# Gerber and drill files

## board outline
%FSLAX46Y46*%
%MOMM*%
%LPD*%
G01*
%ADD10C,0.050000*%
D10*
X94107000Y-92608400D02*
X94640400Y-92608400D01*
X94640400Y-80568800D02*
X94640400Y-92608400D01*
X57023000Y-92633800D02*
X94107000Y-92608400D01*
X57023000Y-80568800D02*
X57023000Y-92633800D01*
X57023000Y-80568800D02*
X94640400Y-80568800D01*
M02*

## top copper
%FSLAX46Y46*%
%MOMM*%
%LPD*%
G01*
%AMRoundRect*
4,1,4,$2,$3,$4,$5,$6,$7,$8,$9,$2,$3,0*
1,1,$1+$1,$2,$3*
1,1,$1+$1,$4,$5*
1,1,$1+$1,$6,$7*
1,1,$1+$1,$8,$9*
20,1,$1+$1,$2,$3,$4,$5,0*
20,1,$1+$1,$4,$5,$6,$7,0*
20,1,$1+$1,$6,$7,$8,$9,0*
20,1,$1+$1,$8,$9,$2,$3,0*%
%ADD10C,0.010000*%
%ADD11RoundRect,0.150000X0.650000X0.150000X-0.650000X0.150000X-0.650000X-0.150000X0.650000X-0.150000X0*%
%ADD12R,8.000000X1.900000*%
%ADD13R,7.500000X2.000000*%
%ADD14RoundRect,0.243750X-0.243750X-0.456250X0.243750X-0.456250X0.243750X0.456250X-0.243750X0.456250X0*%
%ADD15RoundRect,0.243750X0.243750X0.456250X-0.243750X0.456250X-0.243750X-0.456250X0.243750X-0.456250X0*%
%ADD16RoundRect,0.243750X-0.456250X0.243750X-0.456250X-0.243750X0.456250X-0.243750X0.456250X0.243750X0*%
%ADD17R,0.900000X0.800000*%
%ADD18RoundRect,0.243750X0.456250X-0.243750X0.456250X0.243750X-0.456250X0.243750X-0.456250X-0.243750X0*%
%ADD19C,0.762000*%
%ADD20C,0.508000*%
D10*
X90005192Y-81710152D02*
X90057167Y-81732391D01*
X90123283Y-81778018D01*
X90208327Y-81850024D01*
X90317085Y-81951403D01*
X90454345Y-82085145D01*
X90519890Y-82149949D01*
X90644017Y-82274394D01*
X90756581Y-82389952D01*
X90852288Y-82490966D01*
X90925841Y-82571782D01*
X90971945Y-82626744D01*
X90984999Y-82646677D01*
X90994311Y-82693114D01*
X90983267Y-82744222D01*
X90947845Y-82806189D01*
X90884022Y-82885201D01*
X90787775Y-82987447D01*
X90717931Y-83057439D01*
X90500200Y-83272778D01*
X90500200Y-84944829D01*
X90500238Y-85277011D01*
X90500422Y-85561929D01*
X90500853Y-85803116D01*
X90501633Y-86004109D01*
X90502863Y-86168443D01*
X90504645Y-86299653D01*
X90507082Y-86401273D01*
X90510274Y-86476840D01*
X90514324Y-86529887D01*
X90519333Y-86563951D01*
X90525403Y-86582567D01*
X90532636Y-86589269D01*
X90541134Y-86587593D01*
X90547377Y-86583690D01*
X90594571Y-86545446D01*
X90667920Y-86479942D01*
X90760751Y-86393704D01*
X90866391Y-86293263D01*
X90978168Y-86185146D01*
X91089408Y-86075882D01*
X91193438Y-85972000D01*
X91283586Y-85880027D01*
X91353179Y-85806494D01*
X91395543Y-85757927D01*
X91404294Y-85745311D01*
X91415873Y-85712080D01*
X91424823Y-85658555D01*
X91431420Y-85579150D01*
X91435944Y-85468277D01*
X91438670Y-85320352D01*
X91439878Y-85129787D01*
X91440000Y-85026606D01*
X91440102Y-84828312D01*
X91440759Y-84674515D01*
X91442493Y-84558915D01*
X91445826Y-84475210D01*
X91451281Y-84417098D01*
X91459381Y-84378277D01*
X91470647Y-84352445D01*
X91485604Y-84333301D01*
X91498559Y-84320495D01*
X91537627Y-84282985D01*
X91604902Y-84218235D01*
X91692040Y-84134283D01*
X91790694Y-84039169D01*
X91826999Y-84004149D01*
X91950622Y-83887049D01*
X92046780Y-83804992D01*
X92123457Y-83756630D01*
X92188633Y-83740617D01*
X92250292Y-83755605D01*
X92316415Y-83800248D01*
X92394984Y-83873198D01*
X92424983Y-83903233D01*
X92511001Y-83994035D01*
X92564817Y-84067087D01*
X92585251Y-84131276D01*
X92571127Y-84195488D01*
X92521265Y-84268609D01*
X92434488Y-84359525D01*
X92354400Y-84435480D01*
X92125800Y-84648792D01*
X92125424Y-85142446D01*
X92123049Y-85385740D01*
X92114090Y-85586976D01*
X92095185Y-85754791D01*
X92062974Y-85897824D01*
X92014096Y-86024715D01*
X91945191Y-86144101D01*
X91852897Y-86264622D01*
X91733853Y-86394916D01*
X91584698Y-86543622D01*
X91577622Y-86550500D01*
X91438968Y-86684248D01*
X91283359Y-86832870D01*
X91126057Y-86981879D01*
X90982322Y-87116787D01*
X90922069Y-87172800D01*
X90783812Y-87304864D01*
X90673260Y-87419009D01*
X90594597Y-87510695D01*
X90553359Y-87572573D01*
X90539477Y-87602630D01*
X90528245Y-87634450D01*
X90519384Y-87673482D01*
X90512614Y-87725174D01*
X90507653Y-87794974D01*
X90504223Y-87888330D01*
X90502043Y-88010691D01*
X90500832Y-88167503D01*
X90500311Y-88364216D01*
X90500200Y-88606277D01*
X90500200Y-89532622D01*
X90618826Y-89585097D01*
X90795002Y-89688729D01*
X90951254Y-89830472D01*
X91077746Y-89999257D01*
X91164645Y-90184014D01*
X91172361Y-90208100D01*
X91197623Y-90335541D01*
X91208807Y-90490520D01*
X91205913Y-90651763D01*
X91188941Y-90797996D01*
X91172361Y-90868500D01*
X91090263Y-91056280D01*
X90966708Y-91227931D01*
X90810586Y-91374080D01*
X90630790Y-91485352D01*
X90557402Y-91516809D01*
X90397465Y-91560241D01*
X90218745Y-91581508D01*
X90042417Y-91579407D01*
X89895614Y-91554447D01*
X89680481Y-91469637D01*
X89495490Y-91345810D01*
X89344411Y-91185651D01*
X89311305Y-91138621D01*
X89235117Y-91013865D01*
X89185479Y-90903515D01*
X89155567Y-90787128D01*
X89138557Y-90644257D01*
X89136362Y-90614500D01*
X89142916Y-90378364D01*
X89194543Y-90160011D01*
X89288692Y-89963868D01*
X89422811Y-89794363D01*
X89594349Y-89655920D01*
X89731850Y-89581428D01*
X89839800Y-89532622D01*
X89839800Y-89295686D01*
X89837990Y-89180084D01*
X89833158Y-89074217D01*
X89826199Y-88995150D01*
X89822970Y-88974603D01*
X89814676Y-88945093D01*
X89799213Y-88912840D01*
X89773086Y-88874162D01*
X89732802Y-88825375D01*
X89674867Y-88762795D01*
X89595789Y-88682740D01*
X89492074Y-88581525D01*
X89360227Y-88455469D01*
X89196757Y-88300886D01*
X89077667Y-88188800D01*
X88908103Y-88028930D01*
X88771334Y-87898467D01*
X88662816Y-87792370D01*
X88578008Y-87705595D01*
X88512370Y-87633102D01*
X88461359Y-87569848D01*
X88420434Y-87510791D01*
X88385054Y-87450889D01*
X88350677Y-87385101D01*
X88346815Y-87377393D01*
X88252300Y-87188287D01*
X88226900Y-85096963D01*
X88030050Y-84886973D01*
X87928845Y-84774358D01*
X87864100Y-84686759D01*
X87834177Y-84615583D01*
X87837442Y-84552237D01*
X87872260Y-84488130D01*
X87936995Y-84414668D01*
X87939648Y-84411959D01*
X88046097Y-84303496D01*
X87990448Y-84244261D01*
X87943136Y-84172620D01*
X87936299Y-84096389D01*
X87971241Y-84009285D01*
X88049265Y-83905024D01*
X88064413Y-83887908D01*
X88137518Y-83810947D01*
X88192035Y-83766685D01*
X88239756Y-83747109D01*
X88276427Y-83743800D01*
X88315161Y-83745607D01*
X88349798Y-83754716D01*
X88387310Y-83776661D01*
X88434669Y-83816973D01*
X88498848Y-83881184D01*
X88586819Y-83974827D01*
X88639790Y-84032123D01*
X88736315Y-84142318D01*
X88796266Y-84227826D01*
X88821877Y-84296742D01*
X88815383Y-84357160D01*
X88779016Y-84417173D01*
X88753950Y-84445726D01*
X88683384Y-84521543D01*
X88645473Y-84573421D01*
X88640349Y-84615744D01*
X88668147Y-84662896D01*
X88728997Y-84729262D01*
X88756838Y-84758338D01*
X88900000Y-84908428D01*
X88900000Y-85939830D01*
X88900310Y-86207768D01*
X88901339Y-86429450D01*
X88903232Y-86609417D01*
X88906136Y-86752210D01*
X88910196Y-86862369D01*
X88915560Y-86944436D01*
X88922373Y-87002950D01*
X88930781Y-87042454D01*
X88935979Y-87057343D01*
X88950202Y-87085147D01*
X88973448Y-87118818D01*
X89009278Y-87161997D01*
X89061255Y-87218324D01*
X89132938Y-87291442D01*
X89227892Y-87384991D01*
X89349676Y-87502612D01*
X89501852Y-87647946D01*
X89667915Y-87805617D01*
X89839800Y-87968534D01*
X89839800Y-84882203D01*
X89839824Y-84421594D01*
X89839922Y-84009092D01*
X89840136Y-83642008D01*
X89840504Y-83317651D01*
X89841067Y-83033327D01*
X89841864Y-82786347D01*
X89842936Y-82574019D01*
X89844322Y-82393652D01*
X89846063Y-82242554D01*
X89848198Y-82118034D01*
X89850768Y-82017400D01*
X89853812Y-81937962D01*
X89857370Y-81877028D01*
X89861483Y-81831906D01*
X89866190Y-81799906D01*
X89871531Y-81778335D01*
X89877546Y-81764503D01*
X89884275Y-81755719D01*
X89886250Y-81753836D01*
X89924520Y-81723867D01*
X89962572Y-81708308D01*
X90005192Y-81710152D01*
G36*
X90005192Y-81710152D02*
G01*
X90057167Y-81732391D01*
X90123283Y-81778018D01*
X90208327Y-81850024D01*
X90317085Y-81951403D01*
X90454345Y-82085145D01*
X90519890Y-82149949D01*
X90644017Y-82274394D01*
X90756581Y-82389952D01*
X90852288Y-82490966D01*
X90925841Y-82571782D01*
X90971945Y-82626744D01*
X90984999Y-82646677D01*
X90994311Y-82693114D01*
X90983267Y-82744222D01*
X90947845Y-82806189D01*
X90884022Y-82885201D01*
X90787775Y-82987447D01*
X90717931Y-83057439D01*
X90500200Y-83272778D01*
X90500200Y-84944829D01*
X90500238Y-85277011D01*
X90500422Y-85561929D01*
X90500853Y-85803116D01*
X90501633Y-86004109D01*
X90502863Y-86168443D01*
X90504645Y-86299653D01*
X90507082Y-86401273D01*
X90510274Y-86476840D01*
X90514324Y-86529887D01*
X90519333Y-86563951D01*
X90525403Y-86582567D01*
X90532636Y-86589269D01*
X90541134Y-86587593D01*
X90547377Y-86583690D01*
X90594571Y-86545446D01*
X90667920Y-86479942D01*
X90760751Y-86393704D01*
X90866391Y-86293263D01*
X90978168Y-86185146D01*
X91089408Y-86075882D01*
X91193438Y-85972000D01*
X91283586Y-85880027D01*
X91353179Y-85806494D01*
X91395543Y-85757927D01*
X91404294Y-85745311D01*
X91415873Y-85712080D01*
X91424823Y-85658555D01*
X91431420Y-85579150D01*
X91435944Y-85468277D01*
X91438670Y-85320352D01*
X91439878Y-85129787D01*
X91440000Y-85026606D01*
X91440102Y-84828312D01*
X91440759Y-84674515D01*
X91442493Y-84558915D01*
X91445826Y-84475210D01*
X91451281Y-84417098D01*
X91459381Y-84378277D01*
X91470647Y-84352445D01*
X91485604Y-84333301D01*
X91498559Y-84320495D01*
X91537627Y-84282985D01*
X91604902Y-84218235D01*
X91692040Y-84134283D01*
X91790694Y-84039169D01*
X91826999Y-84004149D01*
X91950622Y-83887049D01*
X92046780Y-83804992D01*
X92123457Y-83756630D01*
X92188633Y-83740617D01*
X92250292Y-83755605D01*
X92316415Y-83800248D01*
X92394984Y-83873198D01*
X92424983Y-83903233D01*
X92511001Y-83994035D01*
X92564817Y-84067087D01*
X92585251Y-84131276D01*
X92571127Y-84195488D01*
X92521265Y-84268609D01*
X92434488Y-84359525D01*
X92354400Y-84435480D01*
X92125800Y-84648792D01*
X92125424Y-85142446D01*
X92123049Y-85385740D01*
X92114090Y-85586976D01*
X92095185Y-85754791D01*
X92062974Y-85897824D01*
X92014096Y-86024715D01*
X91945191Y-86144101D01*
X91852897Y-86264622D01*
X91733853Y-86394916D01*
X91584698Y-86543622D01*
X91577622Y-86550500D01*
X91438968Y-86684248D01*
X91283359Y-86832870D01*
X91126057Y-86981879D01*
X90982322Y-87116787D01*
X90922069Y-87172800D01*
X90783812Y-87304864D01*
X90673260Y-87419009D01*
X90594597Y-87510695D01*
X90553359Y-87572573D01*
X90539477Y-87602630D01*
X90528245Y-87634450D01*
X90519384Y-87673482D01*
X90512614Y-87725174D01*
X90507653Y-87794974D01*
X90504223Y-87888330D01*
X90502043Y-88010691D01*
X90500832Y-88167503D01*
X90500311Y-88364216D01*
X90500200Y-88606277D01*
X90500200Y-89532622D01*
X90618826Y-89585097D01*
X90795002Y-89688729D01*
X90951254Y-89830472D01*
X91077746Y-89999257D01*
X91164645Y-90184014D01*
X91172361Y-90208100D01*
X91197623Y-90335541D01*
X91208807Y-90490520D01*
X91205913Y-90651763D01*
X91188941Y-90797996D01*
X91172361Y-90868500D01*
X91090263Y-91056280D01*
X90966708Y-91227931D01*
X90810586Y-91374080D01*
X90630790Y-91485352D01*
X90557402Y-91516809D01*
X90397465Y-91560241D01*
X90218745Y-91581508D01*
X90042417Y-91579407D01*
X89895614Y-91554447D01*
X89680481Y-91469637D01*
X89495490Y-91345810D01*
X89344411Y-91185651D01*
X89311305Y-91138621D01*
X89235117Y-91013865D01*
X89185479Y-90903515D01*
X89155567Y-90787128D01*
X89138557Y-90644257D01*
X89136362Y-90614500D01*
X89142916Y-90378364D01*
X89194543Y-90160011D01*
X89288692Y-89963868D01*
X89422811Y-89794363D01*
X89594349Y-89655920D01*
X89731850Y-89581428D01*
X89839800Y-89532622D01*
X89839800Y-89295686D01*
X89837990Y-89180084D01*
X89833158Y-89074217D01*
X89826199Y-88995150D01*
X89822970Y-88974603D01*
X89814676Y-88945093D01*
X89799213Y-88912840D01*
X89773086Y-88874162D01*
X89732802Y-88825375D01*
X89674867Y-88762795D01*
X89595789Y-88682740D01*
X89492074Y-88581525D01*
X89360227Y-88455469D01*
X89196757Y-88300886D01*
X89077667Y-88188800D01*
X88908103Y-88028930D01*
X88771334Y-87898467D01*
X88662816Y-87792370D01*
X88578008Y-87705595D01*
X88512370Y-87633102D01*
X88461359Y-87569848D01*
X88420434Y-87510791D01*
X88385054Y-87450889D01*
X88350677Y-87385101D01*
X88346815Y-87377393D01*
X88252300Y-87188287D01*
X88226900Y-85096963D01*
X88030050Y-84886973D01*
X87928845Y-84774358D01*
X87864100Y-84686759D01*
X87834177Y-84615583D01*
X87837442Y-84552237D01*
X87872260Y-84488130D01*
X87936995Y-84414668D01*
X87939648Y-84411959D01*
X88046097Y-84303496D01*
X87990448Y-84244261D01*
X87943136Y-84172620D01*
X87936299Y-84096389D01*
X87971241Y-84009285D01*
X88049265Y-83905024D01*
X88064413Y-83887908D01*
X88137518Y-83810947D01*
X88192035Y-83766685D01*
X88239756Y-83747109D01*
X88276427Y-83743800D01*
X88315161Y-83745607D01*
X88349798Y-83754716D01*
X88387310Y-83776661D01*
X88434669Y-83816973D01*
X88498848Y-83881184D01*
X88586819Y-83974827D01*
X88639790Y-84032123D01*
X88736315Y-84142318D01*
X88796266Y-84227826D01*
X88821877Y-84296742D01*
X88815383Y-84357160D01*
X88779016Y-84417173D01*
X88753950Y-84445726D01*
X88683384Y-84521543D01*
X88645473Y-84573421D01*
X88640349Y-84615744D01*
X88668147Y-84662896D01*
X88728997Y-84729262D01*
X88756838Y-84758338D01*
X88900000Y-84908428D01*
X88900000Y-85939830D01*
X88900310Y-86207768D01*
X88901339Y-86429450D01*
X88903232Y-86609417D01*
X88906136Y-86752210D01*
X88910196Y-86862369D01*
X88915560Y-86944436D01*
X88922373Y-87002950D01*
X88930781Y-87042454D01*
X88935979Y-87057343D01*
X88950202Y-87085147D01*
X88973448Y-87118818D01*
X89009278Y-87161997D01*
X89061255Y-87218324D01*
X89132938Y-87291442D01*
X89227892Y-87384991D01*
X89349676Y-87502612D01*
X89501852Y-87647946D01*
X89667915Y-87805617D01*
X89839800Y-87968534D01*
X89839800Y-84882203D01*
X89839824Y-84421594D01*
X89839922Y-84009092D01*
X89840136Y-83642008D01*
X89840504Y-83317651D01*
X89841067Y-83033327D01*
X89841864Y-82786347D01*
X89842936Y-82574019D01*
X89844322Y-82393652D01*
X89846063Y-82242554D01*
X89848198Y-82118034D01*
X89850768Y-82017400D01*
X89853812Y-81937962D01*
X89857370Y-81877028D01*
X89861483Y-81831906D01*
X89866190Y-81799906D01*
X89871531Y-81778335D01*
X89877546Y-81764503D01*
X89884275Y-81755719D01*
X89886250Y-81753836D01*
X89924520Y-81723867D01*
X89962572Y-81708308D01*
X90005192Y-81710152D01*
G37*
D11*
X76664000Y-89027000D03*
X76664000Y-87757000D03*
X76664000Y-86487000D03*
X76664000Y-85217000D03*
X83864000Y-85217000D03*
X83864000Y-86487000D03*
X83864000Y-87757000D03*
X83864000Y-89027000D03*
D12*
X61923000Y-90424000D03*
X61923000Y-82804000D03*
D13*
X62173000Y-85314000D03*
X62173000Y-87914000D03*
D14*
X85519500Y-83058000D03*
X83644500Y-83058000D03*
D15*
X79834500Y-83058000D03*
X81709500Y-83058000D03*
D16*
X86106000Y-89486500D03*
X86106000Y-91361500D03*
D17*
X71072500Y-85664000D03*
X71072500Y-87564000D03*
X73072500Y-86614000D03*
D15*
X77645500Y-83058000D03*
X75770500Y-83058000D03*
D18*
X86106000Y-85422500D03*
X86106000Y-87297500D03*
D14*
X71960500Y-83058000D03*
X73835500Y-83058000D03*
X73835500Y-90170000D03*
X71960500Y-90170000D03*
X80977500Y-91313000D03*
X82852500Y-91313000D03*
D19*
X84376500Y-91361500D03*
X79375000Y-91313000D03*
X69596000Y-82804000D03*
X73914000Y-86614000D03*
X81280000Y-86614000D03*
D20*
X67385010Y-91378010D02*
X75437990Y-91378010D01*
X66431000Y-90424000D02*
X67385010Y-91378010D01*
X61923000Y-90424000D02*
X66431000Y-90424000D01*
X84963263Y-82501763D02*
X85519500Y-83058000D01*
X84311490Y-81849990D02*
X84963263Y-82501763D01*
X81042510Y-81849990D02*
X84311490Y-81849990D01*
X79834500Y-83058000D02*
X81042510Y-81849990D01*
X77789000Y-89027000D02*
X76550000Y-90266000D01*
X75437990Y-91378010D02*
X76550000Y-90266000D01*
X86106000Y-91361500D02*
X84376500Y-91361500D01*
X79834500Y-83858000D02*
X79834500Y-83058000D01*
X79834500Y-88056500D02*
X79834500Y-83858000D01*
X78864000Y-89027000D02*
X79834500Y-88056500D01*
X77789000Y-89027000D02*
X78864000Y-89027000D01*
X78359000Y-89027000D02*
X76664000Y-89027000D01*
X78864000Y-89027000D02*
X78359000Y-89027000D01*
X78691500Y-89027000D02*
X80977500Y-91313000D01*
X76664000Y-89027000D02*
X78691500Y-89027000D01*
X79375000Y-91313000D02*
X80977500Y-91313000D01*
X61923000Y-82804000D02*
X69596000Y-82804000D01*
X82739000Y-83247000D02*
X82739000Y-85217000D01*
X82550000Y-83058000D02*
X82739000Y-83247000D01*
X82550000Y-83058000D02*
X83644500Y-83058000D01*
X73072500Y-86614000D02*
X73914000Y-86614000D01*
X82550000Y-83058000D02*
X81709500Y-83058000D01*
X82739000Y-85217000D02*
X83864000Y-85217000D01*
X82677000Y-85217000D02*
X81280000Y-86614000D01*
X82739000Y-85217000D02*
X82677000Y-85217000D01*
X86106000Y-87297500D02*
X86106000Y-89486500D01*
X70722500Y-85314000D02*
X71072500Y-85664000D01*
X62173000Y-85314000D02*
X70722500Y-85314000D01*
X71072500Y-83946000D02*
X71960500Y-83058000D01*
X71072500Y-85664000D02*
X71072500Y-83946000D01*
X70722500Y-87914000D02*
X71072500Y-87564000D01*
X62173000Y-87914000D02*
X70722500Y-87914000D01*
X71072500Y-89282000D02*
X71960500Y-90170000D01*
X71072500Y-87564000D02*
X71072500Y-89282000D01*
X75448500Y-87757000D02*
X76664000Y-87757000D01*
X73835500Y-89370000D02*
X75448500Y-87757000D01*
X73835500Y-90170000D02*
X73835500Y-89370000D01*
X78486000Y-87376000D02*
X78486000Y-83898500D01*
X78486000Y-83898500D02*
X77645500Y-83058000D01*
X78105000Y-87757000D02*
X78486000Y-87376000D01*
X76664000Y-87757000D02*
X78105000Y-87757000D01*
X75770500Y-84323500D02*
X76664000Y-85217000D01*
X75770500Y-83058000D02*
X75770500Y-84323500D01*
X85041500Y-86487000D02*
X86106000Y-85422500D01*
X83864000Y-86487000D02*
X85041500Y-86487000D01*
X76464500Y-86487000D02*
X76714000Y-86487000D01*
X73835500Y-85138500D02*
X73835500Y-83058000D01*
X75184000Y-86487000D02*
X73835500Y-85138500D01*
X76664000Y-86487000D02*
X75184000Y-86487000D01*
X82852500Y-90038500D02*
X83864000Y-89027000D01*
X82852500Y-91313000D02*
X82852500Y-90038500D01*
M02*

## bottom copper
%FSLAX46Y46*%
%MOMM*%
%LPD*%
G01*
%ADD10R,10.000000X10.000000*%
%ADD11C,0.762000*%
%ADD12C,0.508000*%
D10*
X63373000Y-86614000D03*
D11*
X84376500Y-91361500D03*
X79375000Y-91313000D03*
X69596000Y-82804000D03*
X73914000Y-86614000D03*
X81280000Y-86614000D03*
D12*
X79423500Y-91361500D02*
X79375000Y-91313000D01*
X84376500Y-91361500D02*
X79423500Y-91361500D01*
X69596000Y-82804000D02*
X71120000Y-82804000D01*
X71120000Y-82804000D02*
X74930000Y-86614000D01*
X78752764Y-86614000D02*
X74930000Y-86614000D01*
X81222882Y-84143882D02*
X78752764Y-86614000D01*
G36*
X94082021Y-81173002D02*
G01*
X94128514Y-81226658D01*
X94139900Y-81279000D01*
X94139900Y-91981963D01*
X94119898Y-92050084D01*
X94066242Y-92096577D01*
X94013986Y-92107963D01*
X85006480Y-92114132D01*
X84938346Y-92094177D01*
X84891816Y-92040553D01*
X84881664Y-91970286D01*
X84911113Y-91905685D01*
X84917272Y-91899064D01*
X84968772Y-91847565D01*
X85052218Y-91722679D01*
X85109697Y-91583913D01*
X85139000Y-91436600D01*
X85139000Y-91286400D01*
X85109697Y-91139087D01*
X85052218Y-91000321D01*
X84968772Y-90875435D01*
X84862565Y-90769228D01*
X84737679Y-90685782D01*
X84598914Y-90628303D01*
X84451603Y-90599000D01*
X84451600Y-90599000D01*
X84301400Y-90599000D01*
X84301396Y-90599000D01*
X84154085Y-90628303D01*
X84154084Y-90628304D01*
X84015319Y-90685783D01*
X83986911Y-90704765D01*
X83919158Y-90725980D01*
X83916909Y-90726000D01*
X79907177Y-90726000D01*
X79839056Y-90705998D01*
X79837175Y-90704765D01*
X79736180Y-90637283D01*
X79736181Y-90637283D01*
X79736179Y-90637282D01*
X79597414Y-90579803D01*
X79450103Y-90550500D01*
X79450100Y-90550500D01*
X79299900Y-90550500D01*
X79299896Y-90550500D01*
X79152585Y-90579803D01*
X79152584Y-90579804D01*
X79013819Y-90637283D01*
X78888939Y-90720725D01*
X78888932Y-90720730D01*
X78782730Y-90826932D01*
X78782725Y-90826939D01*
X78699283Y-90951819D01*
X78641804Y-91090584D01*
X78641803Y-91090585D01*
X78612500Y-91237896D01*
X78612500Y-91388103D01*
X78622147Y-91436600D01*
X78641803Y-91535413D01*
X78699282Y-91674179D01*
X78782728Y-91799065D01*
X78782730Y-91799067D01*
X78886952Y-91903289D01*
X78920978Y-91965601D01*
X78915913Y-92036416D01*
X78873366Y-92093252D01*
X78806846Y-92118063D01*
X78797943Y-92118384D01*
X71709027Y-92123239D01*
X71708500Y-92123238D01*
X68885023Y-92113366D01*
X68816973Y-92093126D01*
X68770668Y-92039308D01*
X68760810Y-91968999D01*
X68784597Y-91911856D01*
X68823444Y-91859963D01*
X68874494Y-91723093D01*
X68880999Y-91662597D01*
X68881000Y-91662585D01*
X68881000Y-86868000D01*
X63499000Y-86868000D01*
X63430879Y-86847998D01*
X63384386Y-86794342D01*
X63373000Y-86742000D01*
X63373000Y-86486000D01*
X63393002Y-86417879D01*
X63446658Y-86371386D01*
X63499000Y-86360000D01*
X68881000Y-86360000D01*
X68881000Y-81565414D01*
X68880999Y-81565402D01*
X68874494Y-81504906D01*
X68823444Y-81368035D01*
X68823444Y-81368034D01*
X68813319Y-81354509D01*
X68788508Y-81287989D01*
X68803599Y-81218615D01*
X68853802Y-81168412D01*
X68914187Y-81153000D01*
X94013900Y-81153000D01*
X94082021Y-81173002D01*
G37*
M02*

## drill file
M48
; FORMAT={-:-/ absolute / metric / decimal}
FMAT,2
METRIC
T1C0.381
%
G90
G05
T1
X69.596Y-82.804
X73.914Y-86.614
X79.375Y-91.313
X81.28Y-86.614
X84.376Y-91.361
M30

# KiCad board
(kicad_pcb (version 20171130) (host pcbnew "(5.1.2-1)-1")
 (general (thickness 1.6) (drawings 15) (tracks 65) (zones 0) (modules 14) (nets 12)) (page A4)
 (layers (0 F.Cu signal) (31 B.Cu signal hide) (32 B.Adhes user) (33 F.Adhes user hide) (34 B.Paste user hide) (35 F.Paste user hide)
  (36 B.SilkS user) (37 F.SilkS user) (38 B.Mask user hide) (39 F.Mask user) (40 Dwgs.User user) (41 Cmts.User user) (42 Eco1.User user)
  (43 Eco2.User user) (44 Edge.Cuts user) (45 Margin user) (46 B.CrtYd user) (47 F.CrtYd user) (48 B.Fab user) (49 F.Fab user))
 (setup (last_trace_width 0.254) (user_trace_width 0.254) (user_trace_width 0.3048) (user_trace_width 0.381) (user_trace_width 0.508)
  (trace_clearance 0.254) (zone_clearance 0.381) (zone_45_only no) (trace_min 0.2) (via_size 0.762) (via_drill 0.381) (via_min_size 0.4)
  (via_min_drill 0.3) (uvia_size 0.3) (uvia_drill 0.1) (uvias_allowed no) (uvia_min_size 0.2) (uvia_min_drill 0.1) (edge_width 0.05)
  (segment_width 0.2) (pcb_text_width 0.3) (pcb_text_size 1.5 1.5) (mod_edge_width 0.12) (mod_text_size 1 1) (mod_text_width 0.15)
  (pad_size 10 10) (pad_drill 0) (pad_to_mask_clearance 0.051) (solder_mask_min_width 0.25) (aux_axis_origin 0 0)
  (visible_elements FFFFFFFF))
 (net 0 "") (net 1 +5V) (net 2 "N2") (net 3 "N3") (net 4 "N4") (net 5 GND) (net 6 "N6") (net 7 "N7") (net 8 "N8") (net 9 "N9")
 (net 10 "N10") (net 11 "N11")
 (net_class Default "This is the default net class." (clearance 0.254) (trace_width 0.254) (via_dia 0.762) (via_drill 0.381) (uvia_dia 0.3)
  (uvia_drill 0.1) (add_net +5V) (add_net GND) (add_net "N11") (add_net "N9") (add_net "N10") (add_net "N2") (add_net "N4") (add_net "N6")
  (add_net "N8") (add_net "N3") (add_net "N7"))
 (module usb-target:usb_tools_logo (layer B.Cu) (at 91.567 86.487 180)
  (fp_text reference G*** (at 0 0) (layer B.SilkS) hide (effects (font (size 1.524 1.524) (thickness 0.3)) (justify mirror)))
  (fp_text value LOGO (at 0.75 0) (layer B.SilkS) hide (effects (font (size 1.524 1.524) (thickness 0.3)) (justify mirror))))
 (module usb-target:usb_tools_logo (layer F.Cu) (at 90.17 86.614)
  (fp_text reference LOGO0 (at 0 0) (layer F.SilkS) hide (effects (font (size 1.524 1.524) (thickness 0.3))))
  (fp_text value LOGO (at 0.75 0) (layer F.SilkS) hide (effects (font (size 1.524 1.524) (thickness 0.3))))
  (fp_poly
   (pts (xy -0.164808 -4.903848) (xy -0.112833 -4.881609) (xy -0.046717 -4.835982) (xy 0.038327 -4.763976) (xy 0.147085 -4.662597)
    (xy 0.284345 -4.528855) (xy 0.34989 -4.464051) (xy 0.474017 -4.339606) (xy 0.586581 -4.224048) (xy 0.682288 -4.123034)
    (xy 0.755841 -4.042218) (xy 0.801945 -3.987256) (xy 0.814999 -3.967323) (xy 0.824311 -3.920886) (xy 0.813267 -3.869778)
    (xy 0.777845 -3.807811) (xy 0.714022 -3.728799) (xy 0.617775 -3.626553) (xy 0.547931 -3.556561) (xy 0.3302 -3.341222)
    (xy 0.3302 -1.669171) (xy 0.330238 -1.336989) (xy 0.330422 -1.052071) (xy 0.330853 -0.810884) (xy 0.331633 -0.609891)
    (xy 0.332863 -0.445557) (xy 0.334645 -0.314347) (xy 0.337082 -0.212727) (xy 0.340274 -0.13716) (xy 0.344324 -0.084113)
    (xy 0.349333 -0.050049) (xy 0.355403 -0.031433) (xy 0.362636 -0.024731) (xy 0.371134 -0.026407) (xy 0.377377 -0.03031)
    (xy 0.424571 -0.068554) (xy 0.49792 -0.134058) (xy 0.590751 -0.220296) (xy 0.696391 -0.320737) (xy 0.808168 -0.428854)
    (xy 0.919408 -0.538118) (xy 1.023438 -0.642) (xy 1.113586 -0.733973) (xy 1.183179 -0.807506) (xy 1.225543 -0.856073)
    (xy 1.234294 -0.868689) (xy 1.245873 -0.90192) (xy 1.254823 -0.955445) (xy 1.26142 -1.03485) (xy 1.265944 -1.145723)
    (xy 1.26867 -1.293648) (xy 1.269878 -1.484213) (xy 1.27 -1.587394) (xy 1.270102 -1.785688) (xy 1.270759 -1.939485)
    (xy 1.272493 -2.055085) (xy 1.275826 -2.13879) (xy 1.281281 -2.196902) (xy 1.289381 -2.235723) (xy 1.300647 -2.261555)
    (xy 1.315604 -2.280699) (xy 1.328559 -2.293505) (xy 1.367627 -2.331015) (xy 1.434902 -2.395765) (xy 1.52204 -2.479717)
    (xy 1.620694 -2.574831) (xy 1.656999 -2.609851) (xy 1.780622 -2.726951) (xy 1.87678 -2.809008) (xy 1.953457 -2.85737)
    (xy 2.018633 -2.873383) (xy 2.080292 -2.858395) (xy 2.146415 -2.813752) (xy 2.224984 -2.740802) (xy 2.254983 -2.710767)
    (xy 2.341001 -2.619965) (xy 2.394817 -2.546913) (xy 2.415251 -2.482724) (xy 2.401127 -2.418512) (xy 2.351265 -2.345391)
    (xy 2.264488 -2.254475) (xy 2.1844 -2.17852) (xy 1.9558 -1.965208) (xy 1.955424 -1.471554) (xy 1.953049 -1.22826) (xy 1.94409 -1.027024)
    (xy 1.925185 -0.859209) (xy 1.892974 -0.716176) (xy 1.844096 -0.589285) (xy 1.775191 -0.469899) (xy 1.682897 -0.349378)
    (xy 1.563853 -0.219084) (xy 1.414698 -0.070378) (xy 1.407622 -0.0635) (xy 1.268968 0.070248) (xy 1.113359 0.21887)
    (xy 0.956057 0.367879) (xy 0.812322 0.502787) (xy 0.752069 0.5588) (xy 0.613812 0.690864) (xy 0.50326 0.805009) (xy 0.424597 0.896695)
    (xy 0.383359 0.958573) (xy 0.369477 0.98863) (xy 0.358245 1.02045) (xy 0.349384 1.059482) (xy 0.342614 1.111174) (xy 0.337653 1.180974)
    (xy 0.334223 1.27433) (xy 0.332043 1.396691) (xy 0.330832 1.553503) (xy 0.330311 1.750216) (xy 0.3302 1.992277) (xy 0.3302 2.918622)
    (xy 0.448826 2.971097) (xy 0.625002 3.074729) (xy 0.781254 3.216472) (xy 0.907746 3.385257) (xy 0.994645 3.570014) (xy 1.002361 3.5941)
    (xy 1.027623 3.721541) (xy 1.038807 3.87652) (xy 1.035913 4.037763) (xy 1.018941 4.183996) (xy 1.002361 4.2545) (xy 0.920263 4.44228)
    (xy 0.796708 4.613931) (xy 0.640586 4.76008) (xy 0.46079 4.871352) (xy 0.387402 4.902809) (xy 0.227465 4.946241) (xy 0.048745 4.967508)
    (xy -0.127583 4.965407) (xy -0.274386 4.940447) (xy -0.489519 4.855637) (xy -0.67451 4.73181) (xy -0.825589 4.571651)
    (xy -0.858695 4.524621) (xy -0.934883 4.399865) (xy -0.984521 4.289515) (xy -1.014433 4.173128) (xy -1.031443 4.030257)
    (xy -1.033638 4.0005) (xy -1.027084 3.764364) (xy -0.975457 3.546011) (xy -0.881308 3.349868) (xy -0.747189 3.180363)
    (xy -0.575651 3.04192) (xy -0.43815 2.967428) (xy -0.3302 2.918622) (xy -0.3302 2.681686) (xy -0.33201 2.566084) (xy -0.336842 2.460217)
    (xy -0.343801 2.38115) (xy -0.34703 2.360603) (xy -0.355324 2.331093) (xy -0.370787 2.29884) (xy -0.396914 2.260162)
    (xy -0.437198 2.211375) (xy -0.495133 2.148795) (xy -0.574211 2.06874) (xy -0.677926 1.967525) (xy -0.809773 1.841469)
    (xy -0.973243 1.686886) (xy -1.092333 1.5748) (xy -1.261897 1.41493) (xy -1.398666 1.284467) (xy -1.507184 1.17837)
    (xy -1.591992 1.091595) (xy -1.65763 1.019102) (xy -1.708641 0.955848) (xy -1.749566 0.896791) (xy -1.784946 0.836889)
    (xy -1.819323 0.771101) (xy -1.823185 0.763393) (xy -1.9177 0.574287) (xy -1.9431 -1.517037) (xy -2.13995 -1.727027)
    (xy -2.241155 -1.839642) (xy -2.3059 -1.927241) (xy -2.335823 -1.998417) (xy -2.332558 -2.061763) (xy -2.29774 -2.12587)
    (xy -2.233005 -2.199332) (xy -2.230352 -2.202041) (xy -2.123903 -2.310504) (xy -2.179552 -2.369739) (xy -2.226864 -2.44138)
    (xy -2.233701 -2.517611) (xy -2.198759 -2.604715) (xy -2.120735 -2.708976) (xy -2.105587 -2.726092) (xy -2.032482 -2.803053)
    (xy -1.977965 -2.847315) (xy -1.930244 -2.866891) (xy -1.893573 -2.8702) (xy -1.854839 -2.868393) (xy -1.820202 -2.859284)
    (xy -1.78269 -2.837339) (xy -1.735331 -2.797027) (xy -1.671152 -2.732816) (xy -1.583181 -2.639173) (xy -1.53021 -2.581877)
    (xy -1.433685 -2.471682) (xy -1.373734 -2.386174) (xy -1.348123 -2.317258) (xy -1.354617 -2.25684) (xy -1.390984 -2.196827)
    (xy -1.41605 -2.168274) (xy -1.486616 -2.092457) (xy -1.524527 -2.040579) (xy -1.529651 -1.998256) (xy -1.501853 -1.951104)
    (xy -1.441003 -1.884738) (xy -1.413162 -1.855662) (xy -1.27 -1.705572) (xy -1.27 -0.67417) (xy -1.26969 -0.406232)
    (xy -1.268661 -0.18455) (xy -1.266768 -0.004583) (xy -1.263864 0.13821) (xy -1.259804 0.248369) (xy -1.25444 0.330436)
    (xy -1.247627 0.38895) (xy -1.239219 0.428454) (xy -1.234021 0.443343) (xy -1.219798 0.471147) (xy -1.196552 0.504818)
    (xy -1.160722 0.547997) (xy -1.108745 0.604324) (xy -1.037062 0.677442) (xy -0.942108 0.770991) (xy -0.820324 0.888612)
    (xy -0.668148 1.033946) (xy -0.502085 1.191617) (xy -0.3302 1.354534) (xy -0.3302 -1.731797) (xy -0.330176 -2.192406)
    (xy -0.330078 -2.604908) (xy -0.329864 -2.971992) (xy -0.329496 -3.296349) (xy -0.328933 -3.580673) (xy -0.328136 -3.827653)
    (xy -0.327064 -4.039981) (xy -0.325678 -4.220348) (xy -0.323937 -4.371446) (xy -0.321802 -4.495966) (xy -0.319232 -4.5966)
    (xy -0.316188 -4.676038) (xy -0.31263 -4.736972) (xy -0.308517 -4.782094) (xy -0.30381 -4.814094) (xy -0.298469 -4.835665)
    (xy -0.292454 -4.849497) (xy -0.285725 -4.858281) (xy -0.28375 -4.860164) (xy -0.24548 -4.890133) (xy -0.207428 -4.905692)
    (xy -0.164808 -4.903848))
   (layer F.Cu) (width 0.01)))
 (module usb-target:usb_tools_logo (layer F.Cu) (at 90.17 86.614)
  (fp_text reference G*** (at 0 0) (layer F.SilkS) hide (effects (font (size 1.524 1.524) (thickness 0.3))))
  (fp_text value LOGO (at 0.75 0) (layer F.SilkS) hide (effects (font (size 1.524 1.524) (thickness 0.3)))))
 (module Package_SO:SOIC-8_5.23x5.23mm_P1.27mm (layer F.Cu) (at 80.264 87.122 180)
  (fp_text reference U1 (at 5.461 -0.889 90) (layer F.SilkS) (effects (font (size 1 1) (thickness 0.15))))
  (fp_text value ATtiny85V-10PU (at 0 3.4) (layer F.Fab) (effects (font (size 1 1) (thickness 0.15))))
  (pad 8 smd roundrect (at 3.6 -1.905 180) (size 1.6 0.6) (layers F.Cu F.Paste F.Mask) (roundrect_rratio 0.25) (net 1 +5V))
  (pad 7 smd roundrect (at 3.6 -0.635 180) (size 1.6 0.6) (layers F.Cu F.Paste F.Mask) (roundrect_rratio 0.25) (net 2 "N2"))
  (pad 6 smd roundrect (at 3.6 0.635 180) (size 1.6 0.6) (layers F.Cu F.Paste F.Mask) (roundrect_rratio 0.25) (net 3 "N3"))
  (pad 5 smd roundrect (at 3.6 1.905 180) (size 1.6 0.6) (layers F.Cu F.Paste F.Mask) (roundrect_rratio 0.25) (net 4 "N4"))
  (pad 4 smd roundrect (at -3.6 1.905 180) (size 1.6 0.6) (layers F.Cu F.Paste F.Mask) (roundrect_rratio 0.25) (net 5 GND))
  (pad 3 smd roundrect (at -3.6 0.635 180) (size 1.6 0.6) (layers F.Cu F.Paste F.Mask) (roundrect_rratio 0.25) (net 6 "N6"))
  (pad 2 smd roundrect (at -3.6 -0.635 180) (size 1.6 0.6) (layers F.Cu F.Paste F.Mask) (roundrect_rratio 0.25) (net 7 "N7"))
  (pad 1 smd roundrect (at -3.6 -1.905 180) (size 1.6 0.6) (layers F.Cu F.Paste F.Mask) (roundrect_rratio 0.25) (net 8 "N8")))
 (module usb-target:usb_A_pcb (layer F.Cu) (at 57.023 86.614 270)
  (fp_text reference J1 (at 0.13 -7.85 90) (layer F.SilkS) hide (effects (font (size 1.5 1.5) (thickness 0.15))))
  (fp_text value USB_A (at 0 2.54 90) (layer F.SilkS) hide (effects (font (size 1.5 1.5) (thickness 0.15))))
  (pad 1 connect rect (at 3.81 -4.9 270) (size 1.9 8) (layers F.Cu F.Mask) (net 1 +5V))
  (pad 4 connect rect (at -3.81 -4.9 270) (size 1.9 8) (layers F.Cu F.Mask) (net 5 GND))
  (pad 3 connect rect (at -1.3 -5.15 270) (size 2 7.5) (layers F.Cu F.Mask) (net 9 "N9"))
  (pad 2 connect rect (at 1.3 -5.15 270) (size 2 7.5) (layers F.Cu F.Mask) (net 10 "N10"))
  (pad 5 smd rect (at 0 -6.35 270) (size 10 10) (layers B.Cu B.Mask) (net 5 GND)))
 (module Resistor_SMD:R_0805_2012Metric (layer F.Cu) (at 84.582 83.058)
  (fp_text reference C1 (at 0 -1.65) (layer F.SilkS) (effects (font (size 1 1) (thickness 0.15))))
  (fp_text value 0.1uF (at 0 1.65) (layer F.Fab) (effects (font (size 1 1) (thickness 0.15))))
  (pad 2 smd roundrect (at 0.9375 0) (size 0.975 1.4) (layers F.Cu F.Paste F.Mask) (roundrect_rratio 0.25) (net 1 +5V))
  (pad 1 smd roundrect (at -0.9375 0) (size 0.975 1.4) (layers F.Cu F.Paste F.Mask) (roundrect_rratio 0.25) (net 5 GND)))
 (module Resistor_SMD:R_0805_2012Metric (layer F.Cu) (at 80.772 83.058 180)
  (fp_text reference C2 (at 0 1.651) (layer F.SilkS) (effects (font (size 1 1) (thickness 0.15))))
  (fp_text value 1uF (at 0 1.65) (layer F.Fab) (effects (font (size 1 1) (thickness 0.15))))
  (pad 2 smd roundrect (at 0.9375 0 180) (size 0.975 1.4) (layers F.Cu F.Paste F.Mask) (roundrect_rratio 0.25) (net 1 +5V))
  (pad 1 smd roundrect (at -0.9375 0 180) (size 0.975 1.4) (layers F.Cu F.Paste F.Mask) (roundrect_rratio 0.25) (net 5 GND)))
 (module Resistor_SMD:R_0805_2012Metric (layer F.Cu) (at 86.106 90.424 270)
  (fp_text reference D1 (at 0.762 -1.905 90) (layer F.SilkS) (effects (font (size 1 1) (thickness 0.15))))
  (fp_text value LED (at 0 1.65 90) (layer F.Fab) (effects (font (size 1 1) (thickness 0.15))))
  (pad 1 smd roundrect (at -0.9375 0 270) (size 0.975 1.4) (layers F.Cu F.Paste F.Mask) (roundrect_rratio 0.25) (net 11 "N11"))
  (pad 2 smd roundrect (at 0.9375 0 270) (size 0.975 1.4) (layers F.Cu F.Paste F.Mask) (roundrect_rratio 0.25) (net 1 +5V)))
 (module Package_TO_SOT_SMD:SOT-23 (layer F.Cu) (at 72.0725 86.614)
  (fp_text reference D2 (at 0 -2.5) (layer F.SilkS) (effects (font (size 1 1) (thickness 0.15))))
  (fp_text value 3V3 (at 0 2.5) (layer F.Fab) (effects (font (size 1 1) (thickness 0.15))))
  (pad 1 smd rect (at -1 -0.95) (size 0.9 0.8) (layers F.Cu F.Paste F.Mask) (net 9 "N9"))
  (pad 2 smd rect (at -1 0.95) (size 0.9 0.8) (layers F.Cu F.Paste F.Mask) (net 10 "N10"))
  (pad 3 smd rect (at 1 0) (size 0.9 0.8) (layers F.Cu F.Paste F.Mask) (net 5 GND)))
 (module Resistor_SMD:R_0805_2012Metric (layer F.Cu) (at 76.708 83.058 180)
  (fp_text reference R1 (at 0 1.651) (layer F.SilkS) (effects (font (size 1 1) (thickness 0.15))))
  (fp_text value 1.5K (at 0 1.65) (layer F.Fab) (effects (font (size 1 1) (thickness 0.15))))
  (pad 1 smd roundrect (at -0.9375 0 180) (size 0.975 1.4) (layers F.Cu F.Paste F.Mask) (roundrect_rratio 0.25) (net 2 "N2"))
  (pad 2 smd roundrect (at 0.9375 0 180) (size 0.975 1.4) (layers F.Cu F.Paste F.Mask) (roundrect_rratio 0.25) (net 4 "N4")))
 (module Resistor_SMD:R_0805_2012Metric (layer F.Cu) (at 86.106 86.36 90)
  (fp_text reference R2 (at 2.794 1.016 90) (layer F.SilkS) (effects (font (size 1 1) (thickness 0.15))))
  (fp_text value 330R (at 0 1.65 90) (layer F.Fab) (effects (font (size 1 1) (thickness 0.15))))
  (pad 2 smd roundrect (at 0.9375 0 90) (size 0.975 1.4) (layers F.Cu F.Paste F.Mask) (roundrect_rratio 0.25) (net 6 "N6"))
  (pad 1 smd roundrect (at -0.9375 0 90) (size 0.975 1.4) (layers F.Cu F.Paste F.Mask) (roundrect_rratio 0.25) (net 11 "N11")))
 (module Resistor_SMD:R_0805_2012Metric (layer F.Cu) (at 72.898 83.058)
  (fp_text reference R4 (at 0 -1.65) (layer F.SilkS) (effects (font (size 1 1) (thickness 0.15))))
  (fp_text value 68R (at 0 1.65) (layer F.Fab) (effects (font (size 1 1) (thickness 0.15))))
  (pad 1 smd roundrect (at -0.9375 0) (size 0.975 1.4) (layers F.Cu F.Paste F.Mask) (roundrect_rratio 0.25) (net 9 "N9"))
  (pad 2 smd roundrect (at 0.9375 0) (size 0.975 1.4) (layers F.Cu F.Paste F.Mask) (roundrect_rratio 0.25) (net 3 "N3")))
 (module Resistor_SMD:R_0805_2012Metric (layer F.Cu) (at 72.898 90.17)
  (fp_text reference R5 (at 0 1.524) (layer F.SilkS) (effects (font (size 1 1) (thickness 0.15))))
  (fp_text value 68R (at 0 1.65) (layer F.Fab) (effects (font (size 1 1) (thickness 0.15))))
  (pad 2 smd roundrect (at 0.9375 0) (size 0.975 1.4) (layers F.Cu F.Paste F.Mask) (roundrect_rratio 0.25) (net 2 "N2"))
  (pad 1 smd roundrect (at -0.9375 0) (size 0.975 1.4) (layers F.Cu F.Paste F.Mask) (roundrect_rratio 0.25) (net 10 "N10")))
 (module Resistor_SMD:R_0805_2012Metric (layer F.Cu) (at 81.915 91.313)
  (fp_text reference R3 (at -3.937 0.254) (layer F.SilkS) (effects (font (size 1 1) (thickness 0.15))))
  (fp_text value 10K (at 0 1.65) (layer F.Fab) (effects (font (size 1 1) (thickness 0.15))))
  (pad 1 smd roundrect (at -0.9375 0) (size 0.975 1.4) (layers F.Cu F.Paste F.Mask) (roundrect_rratio 0.25) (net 1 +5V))
  (pad 2 smd roundrect (at 0.9375 0) (size 0.975 1.4) (layers F.Cu F.Paste F.Mask) (roundrect_rratio 0.25) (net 8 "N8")))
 (gr_line (start 94.107 92.6084) (end 94.6404 92.6084) (layer Edge.Cuts) (width 0.05))
 (gr_line (start 94.6404 80.5688) (end 94.6404 92.6084) (layer Edge.Cuts) (width 0.05))
 (gr_line (start 57.023 92.6338) (end 94.107 92.6084) (layer Edge.Cuts) (width 0.05))
 (gr_line (start 57.023 80.5688) (end 57.023 92.6338) (layer Edge.Cuts) (width 0.05))
 (gr_line (start 57.023 80.5688) (end 94.6404 80.5688) (layer Edge.Cuts) (width 0.05))
 (segment (start 67.38501 91.37801) (end 75.43799 91.37801) (width 0.508) (layer F.Cu) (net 1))
 (segment (start 66.431 90.424) (end 67.38501 91.37801) (width 0.508) (layer F.Cu) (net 1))
 (segment (start 61.923 90.424) (end 66.431 90.424) (width 0.508) (layer F.Cu) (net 1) (status 10))
 (segment (start 84.963263 82.501763) (end 85.5195 83.058) (width 0.508) (layer F.Cu) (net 1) (status 20))
 (segment (start 84.31149 81.84999) (end 84.963263 82.501763) (width 0.508) (layer F.Cu) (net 1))
 (segment (start 81.04251 81.84999) (end 84.31149 81.84999) (width 0.508) (layer F.Cu) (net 1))
 (segment (start 79.8345 83.058) (end 81.04251 81.84999) (width 0.508) (layer F.Cu) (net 1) (status 10))
 (segment (start 77.789 89.027) (end 76.55 90.266) (width 0.508) (layer F.Cu) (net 1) (status 10))
 (segment (start 75.43799 91.37801) (end 76.55 90.266) (width 0.508) (layer F.Cu) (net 1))
 (segment (start 86.106 91.3615) (end 84.3765 91.3615) (width 0.508) (layer F.Cu) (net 1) (status 10))
 (segment (start 79.8345 83.858) (end 79.8345 83.058) (width 0.508) (layer F.Cu) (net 1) (status 20))
 (segment (start 79.8345 88.0565) (end 79.8345 83.858) (width 0.508) (layer F.Cu) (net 1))
 (segment (start 78.864 89.027) (end 79.8345 88.0565) (width 0.508) (layer F.Cu) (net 1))
 (segment (start 77.789 89.027) (end 78.864 89.027) (width 0.508) (layer F.Cu) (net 1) (status 10))
 (segment (start 78.359 89.027) (end 76.664 89.027) (width 0.508) (layer F.Cu) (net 1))
 (segment (start 78.864 89.027) (end 78.359 89.027) (width 0.508) (layer F.Cu) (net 1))
 (segment (start 78.6915 89.027) (end 80.9775 91.313) (width 0.508) (layer F.Cu) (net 1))
 (segment (start 76.664 89.027) (end 78.6915 89.027) (width 0.508) (layer F.Cu) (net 1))
 (via (at 84.3765 91.3615) (size 0.762) (drill 0.381) (layers F.Cu B.Cu) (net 1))
 (via (at 79.375 91.313) (size 0.762) (drill 0.381) (layers F.Cu B.Cu) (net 1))
 (segment (start 79.4235 91.3615) (end 79.375 91.313) (width 0.508) (layer B.Cu) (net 1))
 (segment (start 84.3765 91.3615) (end 79.4235 91.3615) (width 0.508) (layer B.Cu) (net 1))
 (segment (start 79.375 91.313) (end 80.9775 91.313) (width 0.508) (layer F.Cu) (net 1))
 (via (at 69.596 82.804) (size 0.762) (drill 0.381) (layers F.Cu B.Cu) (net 5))
 (segment (start 61.923 82.804) (end 69.596 82.804) (width 0.508) (layer F.Cu) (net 5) (status 10))
 (segment (start 69.596 82.804) (end 71.12 82.804) (width 0.508) (layer B.Cu) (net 5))
 (segment (start 71.12 82.804) (end 74.93 86.614) (width 0.508) (layer B.Cu) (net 5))
 (segment (start 82.739 83.247) (end 82.739 85.217) (width 0.508) (layer F.Cu) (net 5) (status 20))
 (segment (start 82.55 83.058) (end 82.739 83.247) (width 0.508) (layer F.Cu) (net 5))
 (segment (start 82.55 83.058) (end 83.6445 83.058) (width 0.508) (layer F.Cu) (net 5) (status 20))
 (segment (start 78.752764 86.614) (end 74.93 86.614) (width 0.508) (layer B.Cu) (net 5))
 (segment (start 81.222882 84.143882) (end 78.752764 86.614) (width 0.508) (layer B.Cu) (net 5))
 (via (at 73.914 86.614) (size 0.762) (drill 0.381) (layers F.Cu B.Cu) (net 5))
 (segment (start 73.0725 86.614) (end 73.914 86.614) (width 0.508) (layer F.Cu) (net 5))
 (segment (start 82.55 83.058) (end 81.7095 83.058) (width 0.508) (layer F.Cu) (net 5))
 (segment (start 82.739 85.217) (end 83.864 85.217) (width 0.508) (layer F.Cu) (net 5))
 (via (at 81.28 86.614) (size 0.762) (drill 0.381) (layers F.Cu B.Cu) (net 5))
 (segment (start 82.677 85.217) (end 81.28 86.614) (width 0.508) (layer F.Cu) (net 5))
 (segment (start 82.739 85.217) (end 82.677 85.217) (width 0.508) (layer F.Cu) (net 5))
 (segment (start 86.106 87.2975) (end 86.106 89.4865) (width 0.508) (layer F.Cu) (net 11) (status 30))
 (segment (start 70.7225 85.314) (end 71.0725 85.664) (width 0.508) (layer F.Cu) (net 9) (status 30))
 (segment (start 62.173 85.314) (end 70.7225 85.314) (width 0.508) (layer F.Cu) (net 9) (status 30))
 (segment (start 71.0725 83.946) (end 71.9605 83.058) (width 0.508) (layer F.Cu) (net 9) (status 20))
 (segment (start 71.0725 85.664) (end 71.0725 83.946) (width 0.508) (layer F.Cu) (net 9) (status 10))
 (segment (start 70.7225 87.914) (end 71.0725 87.564) (width 0.508) (layer F.Cu) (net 10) (status 30))
 (segment (start 62.173 87.914) (end 70.7225 87.914) (width 0.508) (layer F.Cu) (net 10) (status 30))
 (segment (start 71.0725 89.282) (end 71.9605 90.17) (width 0.508) (layer F.Cu) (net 10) (status 20))
 (segment (start 71.0725 87.564) (end 71.0725 89.282) (width 0.508) (layer F.Cu) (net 10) (status 10))
 (segment (start 75.4485 87.757) (end 76.664 87.757) (width 0.508) (layer F.Cu) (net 2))
 (segment (start 73.8355 89.37) (end 75.4485 87.757) (width 0.508) (layer F.Cu) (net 2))
 (segment (start 73.8355 90.17) (end 73.8355 89.37) (width 0.508) (layer F.Cu) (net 2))
 (segment (start 78.486 87.376) (end 78.486 83.8985) (width 0.508) (layer F.Cu) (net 2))
 (segment (start 78.486 83.8985) (end 77.6455 83.058) (width 0.508) (layer F.Cu) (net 2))
 (segment (start 78.105 87.757) (end 78.486 87.376) (width 0.508) (layer F.Cu) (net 2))
 (segment (start 76.664 87.757) (end 78.105 87.757) (width 0.508) (layer F.Cu) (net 2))
 (segment (start 75.7705 84.3235) (end 76.664 85.217) (width 0.508) (layer F.Cu) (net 4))
 (segment (start 75.7705 83.058) (end 75.7705 84.3235) (width 0.508) (layer F.Cu) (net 4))
 (segment (start 85.0415 86.487) (end 86.106 85.4225) (width 0.508) (layer F.Cu) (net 6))
 (segment (start 83.864 86.487) (end 85.0415 86.487) (width 0.508) (layer F.Cu) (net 6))
 (segment (start 76.4645 86.487) (end 76.714 86.487) (width 0.508) (layer F.Cu) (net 3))
 (segment (start 73.8355 85.1385) (end 73.8355 83.058) (width 0.508) (layer F.Cu) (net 3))
 (segment (start 75.184 86.487) (end 73.8355 85.1385) (width 0.508) (layer F.Cu) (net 3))
 (segment (start 76.664 86.487) (end 75.184 86.487) (width 0.508) (layer F.Cu) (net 3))
 (segment (start 82.8525 90.0385) (end 83.864 89.027) (width 0.508) (layer F.Cu) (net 8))
 (segment (start 82.8525 91.313) (end 82.8525 90.0385) (width 0.508) (layer F.Cu) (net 8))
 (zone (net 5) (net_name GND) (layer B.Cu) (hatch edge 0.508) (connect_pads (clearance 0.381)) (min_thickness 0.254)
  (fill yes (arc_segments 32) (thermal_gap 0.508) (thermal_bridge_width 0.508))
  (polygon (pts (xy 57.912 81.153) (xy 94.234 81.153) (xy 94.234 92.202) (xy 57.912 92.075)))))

